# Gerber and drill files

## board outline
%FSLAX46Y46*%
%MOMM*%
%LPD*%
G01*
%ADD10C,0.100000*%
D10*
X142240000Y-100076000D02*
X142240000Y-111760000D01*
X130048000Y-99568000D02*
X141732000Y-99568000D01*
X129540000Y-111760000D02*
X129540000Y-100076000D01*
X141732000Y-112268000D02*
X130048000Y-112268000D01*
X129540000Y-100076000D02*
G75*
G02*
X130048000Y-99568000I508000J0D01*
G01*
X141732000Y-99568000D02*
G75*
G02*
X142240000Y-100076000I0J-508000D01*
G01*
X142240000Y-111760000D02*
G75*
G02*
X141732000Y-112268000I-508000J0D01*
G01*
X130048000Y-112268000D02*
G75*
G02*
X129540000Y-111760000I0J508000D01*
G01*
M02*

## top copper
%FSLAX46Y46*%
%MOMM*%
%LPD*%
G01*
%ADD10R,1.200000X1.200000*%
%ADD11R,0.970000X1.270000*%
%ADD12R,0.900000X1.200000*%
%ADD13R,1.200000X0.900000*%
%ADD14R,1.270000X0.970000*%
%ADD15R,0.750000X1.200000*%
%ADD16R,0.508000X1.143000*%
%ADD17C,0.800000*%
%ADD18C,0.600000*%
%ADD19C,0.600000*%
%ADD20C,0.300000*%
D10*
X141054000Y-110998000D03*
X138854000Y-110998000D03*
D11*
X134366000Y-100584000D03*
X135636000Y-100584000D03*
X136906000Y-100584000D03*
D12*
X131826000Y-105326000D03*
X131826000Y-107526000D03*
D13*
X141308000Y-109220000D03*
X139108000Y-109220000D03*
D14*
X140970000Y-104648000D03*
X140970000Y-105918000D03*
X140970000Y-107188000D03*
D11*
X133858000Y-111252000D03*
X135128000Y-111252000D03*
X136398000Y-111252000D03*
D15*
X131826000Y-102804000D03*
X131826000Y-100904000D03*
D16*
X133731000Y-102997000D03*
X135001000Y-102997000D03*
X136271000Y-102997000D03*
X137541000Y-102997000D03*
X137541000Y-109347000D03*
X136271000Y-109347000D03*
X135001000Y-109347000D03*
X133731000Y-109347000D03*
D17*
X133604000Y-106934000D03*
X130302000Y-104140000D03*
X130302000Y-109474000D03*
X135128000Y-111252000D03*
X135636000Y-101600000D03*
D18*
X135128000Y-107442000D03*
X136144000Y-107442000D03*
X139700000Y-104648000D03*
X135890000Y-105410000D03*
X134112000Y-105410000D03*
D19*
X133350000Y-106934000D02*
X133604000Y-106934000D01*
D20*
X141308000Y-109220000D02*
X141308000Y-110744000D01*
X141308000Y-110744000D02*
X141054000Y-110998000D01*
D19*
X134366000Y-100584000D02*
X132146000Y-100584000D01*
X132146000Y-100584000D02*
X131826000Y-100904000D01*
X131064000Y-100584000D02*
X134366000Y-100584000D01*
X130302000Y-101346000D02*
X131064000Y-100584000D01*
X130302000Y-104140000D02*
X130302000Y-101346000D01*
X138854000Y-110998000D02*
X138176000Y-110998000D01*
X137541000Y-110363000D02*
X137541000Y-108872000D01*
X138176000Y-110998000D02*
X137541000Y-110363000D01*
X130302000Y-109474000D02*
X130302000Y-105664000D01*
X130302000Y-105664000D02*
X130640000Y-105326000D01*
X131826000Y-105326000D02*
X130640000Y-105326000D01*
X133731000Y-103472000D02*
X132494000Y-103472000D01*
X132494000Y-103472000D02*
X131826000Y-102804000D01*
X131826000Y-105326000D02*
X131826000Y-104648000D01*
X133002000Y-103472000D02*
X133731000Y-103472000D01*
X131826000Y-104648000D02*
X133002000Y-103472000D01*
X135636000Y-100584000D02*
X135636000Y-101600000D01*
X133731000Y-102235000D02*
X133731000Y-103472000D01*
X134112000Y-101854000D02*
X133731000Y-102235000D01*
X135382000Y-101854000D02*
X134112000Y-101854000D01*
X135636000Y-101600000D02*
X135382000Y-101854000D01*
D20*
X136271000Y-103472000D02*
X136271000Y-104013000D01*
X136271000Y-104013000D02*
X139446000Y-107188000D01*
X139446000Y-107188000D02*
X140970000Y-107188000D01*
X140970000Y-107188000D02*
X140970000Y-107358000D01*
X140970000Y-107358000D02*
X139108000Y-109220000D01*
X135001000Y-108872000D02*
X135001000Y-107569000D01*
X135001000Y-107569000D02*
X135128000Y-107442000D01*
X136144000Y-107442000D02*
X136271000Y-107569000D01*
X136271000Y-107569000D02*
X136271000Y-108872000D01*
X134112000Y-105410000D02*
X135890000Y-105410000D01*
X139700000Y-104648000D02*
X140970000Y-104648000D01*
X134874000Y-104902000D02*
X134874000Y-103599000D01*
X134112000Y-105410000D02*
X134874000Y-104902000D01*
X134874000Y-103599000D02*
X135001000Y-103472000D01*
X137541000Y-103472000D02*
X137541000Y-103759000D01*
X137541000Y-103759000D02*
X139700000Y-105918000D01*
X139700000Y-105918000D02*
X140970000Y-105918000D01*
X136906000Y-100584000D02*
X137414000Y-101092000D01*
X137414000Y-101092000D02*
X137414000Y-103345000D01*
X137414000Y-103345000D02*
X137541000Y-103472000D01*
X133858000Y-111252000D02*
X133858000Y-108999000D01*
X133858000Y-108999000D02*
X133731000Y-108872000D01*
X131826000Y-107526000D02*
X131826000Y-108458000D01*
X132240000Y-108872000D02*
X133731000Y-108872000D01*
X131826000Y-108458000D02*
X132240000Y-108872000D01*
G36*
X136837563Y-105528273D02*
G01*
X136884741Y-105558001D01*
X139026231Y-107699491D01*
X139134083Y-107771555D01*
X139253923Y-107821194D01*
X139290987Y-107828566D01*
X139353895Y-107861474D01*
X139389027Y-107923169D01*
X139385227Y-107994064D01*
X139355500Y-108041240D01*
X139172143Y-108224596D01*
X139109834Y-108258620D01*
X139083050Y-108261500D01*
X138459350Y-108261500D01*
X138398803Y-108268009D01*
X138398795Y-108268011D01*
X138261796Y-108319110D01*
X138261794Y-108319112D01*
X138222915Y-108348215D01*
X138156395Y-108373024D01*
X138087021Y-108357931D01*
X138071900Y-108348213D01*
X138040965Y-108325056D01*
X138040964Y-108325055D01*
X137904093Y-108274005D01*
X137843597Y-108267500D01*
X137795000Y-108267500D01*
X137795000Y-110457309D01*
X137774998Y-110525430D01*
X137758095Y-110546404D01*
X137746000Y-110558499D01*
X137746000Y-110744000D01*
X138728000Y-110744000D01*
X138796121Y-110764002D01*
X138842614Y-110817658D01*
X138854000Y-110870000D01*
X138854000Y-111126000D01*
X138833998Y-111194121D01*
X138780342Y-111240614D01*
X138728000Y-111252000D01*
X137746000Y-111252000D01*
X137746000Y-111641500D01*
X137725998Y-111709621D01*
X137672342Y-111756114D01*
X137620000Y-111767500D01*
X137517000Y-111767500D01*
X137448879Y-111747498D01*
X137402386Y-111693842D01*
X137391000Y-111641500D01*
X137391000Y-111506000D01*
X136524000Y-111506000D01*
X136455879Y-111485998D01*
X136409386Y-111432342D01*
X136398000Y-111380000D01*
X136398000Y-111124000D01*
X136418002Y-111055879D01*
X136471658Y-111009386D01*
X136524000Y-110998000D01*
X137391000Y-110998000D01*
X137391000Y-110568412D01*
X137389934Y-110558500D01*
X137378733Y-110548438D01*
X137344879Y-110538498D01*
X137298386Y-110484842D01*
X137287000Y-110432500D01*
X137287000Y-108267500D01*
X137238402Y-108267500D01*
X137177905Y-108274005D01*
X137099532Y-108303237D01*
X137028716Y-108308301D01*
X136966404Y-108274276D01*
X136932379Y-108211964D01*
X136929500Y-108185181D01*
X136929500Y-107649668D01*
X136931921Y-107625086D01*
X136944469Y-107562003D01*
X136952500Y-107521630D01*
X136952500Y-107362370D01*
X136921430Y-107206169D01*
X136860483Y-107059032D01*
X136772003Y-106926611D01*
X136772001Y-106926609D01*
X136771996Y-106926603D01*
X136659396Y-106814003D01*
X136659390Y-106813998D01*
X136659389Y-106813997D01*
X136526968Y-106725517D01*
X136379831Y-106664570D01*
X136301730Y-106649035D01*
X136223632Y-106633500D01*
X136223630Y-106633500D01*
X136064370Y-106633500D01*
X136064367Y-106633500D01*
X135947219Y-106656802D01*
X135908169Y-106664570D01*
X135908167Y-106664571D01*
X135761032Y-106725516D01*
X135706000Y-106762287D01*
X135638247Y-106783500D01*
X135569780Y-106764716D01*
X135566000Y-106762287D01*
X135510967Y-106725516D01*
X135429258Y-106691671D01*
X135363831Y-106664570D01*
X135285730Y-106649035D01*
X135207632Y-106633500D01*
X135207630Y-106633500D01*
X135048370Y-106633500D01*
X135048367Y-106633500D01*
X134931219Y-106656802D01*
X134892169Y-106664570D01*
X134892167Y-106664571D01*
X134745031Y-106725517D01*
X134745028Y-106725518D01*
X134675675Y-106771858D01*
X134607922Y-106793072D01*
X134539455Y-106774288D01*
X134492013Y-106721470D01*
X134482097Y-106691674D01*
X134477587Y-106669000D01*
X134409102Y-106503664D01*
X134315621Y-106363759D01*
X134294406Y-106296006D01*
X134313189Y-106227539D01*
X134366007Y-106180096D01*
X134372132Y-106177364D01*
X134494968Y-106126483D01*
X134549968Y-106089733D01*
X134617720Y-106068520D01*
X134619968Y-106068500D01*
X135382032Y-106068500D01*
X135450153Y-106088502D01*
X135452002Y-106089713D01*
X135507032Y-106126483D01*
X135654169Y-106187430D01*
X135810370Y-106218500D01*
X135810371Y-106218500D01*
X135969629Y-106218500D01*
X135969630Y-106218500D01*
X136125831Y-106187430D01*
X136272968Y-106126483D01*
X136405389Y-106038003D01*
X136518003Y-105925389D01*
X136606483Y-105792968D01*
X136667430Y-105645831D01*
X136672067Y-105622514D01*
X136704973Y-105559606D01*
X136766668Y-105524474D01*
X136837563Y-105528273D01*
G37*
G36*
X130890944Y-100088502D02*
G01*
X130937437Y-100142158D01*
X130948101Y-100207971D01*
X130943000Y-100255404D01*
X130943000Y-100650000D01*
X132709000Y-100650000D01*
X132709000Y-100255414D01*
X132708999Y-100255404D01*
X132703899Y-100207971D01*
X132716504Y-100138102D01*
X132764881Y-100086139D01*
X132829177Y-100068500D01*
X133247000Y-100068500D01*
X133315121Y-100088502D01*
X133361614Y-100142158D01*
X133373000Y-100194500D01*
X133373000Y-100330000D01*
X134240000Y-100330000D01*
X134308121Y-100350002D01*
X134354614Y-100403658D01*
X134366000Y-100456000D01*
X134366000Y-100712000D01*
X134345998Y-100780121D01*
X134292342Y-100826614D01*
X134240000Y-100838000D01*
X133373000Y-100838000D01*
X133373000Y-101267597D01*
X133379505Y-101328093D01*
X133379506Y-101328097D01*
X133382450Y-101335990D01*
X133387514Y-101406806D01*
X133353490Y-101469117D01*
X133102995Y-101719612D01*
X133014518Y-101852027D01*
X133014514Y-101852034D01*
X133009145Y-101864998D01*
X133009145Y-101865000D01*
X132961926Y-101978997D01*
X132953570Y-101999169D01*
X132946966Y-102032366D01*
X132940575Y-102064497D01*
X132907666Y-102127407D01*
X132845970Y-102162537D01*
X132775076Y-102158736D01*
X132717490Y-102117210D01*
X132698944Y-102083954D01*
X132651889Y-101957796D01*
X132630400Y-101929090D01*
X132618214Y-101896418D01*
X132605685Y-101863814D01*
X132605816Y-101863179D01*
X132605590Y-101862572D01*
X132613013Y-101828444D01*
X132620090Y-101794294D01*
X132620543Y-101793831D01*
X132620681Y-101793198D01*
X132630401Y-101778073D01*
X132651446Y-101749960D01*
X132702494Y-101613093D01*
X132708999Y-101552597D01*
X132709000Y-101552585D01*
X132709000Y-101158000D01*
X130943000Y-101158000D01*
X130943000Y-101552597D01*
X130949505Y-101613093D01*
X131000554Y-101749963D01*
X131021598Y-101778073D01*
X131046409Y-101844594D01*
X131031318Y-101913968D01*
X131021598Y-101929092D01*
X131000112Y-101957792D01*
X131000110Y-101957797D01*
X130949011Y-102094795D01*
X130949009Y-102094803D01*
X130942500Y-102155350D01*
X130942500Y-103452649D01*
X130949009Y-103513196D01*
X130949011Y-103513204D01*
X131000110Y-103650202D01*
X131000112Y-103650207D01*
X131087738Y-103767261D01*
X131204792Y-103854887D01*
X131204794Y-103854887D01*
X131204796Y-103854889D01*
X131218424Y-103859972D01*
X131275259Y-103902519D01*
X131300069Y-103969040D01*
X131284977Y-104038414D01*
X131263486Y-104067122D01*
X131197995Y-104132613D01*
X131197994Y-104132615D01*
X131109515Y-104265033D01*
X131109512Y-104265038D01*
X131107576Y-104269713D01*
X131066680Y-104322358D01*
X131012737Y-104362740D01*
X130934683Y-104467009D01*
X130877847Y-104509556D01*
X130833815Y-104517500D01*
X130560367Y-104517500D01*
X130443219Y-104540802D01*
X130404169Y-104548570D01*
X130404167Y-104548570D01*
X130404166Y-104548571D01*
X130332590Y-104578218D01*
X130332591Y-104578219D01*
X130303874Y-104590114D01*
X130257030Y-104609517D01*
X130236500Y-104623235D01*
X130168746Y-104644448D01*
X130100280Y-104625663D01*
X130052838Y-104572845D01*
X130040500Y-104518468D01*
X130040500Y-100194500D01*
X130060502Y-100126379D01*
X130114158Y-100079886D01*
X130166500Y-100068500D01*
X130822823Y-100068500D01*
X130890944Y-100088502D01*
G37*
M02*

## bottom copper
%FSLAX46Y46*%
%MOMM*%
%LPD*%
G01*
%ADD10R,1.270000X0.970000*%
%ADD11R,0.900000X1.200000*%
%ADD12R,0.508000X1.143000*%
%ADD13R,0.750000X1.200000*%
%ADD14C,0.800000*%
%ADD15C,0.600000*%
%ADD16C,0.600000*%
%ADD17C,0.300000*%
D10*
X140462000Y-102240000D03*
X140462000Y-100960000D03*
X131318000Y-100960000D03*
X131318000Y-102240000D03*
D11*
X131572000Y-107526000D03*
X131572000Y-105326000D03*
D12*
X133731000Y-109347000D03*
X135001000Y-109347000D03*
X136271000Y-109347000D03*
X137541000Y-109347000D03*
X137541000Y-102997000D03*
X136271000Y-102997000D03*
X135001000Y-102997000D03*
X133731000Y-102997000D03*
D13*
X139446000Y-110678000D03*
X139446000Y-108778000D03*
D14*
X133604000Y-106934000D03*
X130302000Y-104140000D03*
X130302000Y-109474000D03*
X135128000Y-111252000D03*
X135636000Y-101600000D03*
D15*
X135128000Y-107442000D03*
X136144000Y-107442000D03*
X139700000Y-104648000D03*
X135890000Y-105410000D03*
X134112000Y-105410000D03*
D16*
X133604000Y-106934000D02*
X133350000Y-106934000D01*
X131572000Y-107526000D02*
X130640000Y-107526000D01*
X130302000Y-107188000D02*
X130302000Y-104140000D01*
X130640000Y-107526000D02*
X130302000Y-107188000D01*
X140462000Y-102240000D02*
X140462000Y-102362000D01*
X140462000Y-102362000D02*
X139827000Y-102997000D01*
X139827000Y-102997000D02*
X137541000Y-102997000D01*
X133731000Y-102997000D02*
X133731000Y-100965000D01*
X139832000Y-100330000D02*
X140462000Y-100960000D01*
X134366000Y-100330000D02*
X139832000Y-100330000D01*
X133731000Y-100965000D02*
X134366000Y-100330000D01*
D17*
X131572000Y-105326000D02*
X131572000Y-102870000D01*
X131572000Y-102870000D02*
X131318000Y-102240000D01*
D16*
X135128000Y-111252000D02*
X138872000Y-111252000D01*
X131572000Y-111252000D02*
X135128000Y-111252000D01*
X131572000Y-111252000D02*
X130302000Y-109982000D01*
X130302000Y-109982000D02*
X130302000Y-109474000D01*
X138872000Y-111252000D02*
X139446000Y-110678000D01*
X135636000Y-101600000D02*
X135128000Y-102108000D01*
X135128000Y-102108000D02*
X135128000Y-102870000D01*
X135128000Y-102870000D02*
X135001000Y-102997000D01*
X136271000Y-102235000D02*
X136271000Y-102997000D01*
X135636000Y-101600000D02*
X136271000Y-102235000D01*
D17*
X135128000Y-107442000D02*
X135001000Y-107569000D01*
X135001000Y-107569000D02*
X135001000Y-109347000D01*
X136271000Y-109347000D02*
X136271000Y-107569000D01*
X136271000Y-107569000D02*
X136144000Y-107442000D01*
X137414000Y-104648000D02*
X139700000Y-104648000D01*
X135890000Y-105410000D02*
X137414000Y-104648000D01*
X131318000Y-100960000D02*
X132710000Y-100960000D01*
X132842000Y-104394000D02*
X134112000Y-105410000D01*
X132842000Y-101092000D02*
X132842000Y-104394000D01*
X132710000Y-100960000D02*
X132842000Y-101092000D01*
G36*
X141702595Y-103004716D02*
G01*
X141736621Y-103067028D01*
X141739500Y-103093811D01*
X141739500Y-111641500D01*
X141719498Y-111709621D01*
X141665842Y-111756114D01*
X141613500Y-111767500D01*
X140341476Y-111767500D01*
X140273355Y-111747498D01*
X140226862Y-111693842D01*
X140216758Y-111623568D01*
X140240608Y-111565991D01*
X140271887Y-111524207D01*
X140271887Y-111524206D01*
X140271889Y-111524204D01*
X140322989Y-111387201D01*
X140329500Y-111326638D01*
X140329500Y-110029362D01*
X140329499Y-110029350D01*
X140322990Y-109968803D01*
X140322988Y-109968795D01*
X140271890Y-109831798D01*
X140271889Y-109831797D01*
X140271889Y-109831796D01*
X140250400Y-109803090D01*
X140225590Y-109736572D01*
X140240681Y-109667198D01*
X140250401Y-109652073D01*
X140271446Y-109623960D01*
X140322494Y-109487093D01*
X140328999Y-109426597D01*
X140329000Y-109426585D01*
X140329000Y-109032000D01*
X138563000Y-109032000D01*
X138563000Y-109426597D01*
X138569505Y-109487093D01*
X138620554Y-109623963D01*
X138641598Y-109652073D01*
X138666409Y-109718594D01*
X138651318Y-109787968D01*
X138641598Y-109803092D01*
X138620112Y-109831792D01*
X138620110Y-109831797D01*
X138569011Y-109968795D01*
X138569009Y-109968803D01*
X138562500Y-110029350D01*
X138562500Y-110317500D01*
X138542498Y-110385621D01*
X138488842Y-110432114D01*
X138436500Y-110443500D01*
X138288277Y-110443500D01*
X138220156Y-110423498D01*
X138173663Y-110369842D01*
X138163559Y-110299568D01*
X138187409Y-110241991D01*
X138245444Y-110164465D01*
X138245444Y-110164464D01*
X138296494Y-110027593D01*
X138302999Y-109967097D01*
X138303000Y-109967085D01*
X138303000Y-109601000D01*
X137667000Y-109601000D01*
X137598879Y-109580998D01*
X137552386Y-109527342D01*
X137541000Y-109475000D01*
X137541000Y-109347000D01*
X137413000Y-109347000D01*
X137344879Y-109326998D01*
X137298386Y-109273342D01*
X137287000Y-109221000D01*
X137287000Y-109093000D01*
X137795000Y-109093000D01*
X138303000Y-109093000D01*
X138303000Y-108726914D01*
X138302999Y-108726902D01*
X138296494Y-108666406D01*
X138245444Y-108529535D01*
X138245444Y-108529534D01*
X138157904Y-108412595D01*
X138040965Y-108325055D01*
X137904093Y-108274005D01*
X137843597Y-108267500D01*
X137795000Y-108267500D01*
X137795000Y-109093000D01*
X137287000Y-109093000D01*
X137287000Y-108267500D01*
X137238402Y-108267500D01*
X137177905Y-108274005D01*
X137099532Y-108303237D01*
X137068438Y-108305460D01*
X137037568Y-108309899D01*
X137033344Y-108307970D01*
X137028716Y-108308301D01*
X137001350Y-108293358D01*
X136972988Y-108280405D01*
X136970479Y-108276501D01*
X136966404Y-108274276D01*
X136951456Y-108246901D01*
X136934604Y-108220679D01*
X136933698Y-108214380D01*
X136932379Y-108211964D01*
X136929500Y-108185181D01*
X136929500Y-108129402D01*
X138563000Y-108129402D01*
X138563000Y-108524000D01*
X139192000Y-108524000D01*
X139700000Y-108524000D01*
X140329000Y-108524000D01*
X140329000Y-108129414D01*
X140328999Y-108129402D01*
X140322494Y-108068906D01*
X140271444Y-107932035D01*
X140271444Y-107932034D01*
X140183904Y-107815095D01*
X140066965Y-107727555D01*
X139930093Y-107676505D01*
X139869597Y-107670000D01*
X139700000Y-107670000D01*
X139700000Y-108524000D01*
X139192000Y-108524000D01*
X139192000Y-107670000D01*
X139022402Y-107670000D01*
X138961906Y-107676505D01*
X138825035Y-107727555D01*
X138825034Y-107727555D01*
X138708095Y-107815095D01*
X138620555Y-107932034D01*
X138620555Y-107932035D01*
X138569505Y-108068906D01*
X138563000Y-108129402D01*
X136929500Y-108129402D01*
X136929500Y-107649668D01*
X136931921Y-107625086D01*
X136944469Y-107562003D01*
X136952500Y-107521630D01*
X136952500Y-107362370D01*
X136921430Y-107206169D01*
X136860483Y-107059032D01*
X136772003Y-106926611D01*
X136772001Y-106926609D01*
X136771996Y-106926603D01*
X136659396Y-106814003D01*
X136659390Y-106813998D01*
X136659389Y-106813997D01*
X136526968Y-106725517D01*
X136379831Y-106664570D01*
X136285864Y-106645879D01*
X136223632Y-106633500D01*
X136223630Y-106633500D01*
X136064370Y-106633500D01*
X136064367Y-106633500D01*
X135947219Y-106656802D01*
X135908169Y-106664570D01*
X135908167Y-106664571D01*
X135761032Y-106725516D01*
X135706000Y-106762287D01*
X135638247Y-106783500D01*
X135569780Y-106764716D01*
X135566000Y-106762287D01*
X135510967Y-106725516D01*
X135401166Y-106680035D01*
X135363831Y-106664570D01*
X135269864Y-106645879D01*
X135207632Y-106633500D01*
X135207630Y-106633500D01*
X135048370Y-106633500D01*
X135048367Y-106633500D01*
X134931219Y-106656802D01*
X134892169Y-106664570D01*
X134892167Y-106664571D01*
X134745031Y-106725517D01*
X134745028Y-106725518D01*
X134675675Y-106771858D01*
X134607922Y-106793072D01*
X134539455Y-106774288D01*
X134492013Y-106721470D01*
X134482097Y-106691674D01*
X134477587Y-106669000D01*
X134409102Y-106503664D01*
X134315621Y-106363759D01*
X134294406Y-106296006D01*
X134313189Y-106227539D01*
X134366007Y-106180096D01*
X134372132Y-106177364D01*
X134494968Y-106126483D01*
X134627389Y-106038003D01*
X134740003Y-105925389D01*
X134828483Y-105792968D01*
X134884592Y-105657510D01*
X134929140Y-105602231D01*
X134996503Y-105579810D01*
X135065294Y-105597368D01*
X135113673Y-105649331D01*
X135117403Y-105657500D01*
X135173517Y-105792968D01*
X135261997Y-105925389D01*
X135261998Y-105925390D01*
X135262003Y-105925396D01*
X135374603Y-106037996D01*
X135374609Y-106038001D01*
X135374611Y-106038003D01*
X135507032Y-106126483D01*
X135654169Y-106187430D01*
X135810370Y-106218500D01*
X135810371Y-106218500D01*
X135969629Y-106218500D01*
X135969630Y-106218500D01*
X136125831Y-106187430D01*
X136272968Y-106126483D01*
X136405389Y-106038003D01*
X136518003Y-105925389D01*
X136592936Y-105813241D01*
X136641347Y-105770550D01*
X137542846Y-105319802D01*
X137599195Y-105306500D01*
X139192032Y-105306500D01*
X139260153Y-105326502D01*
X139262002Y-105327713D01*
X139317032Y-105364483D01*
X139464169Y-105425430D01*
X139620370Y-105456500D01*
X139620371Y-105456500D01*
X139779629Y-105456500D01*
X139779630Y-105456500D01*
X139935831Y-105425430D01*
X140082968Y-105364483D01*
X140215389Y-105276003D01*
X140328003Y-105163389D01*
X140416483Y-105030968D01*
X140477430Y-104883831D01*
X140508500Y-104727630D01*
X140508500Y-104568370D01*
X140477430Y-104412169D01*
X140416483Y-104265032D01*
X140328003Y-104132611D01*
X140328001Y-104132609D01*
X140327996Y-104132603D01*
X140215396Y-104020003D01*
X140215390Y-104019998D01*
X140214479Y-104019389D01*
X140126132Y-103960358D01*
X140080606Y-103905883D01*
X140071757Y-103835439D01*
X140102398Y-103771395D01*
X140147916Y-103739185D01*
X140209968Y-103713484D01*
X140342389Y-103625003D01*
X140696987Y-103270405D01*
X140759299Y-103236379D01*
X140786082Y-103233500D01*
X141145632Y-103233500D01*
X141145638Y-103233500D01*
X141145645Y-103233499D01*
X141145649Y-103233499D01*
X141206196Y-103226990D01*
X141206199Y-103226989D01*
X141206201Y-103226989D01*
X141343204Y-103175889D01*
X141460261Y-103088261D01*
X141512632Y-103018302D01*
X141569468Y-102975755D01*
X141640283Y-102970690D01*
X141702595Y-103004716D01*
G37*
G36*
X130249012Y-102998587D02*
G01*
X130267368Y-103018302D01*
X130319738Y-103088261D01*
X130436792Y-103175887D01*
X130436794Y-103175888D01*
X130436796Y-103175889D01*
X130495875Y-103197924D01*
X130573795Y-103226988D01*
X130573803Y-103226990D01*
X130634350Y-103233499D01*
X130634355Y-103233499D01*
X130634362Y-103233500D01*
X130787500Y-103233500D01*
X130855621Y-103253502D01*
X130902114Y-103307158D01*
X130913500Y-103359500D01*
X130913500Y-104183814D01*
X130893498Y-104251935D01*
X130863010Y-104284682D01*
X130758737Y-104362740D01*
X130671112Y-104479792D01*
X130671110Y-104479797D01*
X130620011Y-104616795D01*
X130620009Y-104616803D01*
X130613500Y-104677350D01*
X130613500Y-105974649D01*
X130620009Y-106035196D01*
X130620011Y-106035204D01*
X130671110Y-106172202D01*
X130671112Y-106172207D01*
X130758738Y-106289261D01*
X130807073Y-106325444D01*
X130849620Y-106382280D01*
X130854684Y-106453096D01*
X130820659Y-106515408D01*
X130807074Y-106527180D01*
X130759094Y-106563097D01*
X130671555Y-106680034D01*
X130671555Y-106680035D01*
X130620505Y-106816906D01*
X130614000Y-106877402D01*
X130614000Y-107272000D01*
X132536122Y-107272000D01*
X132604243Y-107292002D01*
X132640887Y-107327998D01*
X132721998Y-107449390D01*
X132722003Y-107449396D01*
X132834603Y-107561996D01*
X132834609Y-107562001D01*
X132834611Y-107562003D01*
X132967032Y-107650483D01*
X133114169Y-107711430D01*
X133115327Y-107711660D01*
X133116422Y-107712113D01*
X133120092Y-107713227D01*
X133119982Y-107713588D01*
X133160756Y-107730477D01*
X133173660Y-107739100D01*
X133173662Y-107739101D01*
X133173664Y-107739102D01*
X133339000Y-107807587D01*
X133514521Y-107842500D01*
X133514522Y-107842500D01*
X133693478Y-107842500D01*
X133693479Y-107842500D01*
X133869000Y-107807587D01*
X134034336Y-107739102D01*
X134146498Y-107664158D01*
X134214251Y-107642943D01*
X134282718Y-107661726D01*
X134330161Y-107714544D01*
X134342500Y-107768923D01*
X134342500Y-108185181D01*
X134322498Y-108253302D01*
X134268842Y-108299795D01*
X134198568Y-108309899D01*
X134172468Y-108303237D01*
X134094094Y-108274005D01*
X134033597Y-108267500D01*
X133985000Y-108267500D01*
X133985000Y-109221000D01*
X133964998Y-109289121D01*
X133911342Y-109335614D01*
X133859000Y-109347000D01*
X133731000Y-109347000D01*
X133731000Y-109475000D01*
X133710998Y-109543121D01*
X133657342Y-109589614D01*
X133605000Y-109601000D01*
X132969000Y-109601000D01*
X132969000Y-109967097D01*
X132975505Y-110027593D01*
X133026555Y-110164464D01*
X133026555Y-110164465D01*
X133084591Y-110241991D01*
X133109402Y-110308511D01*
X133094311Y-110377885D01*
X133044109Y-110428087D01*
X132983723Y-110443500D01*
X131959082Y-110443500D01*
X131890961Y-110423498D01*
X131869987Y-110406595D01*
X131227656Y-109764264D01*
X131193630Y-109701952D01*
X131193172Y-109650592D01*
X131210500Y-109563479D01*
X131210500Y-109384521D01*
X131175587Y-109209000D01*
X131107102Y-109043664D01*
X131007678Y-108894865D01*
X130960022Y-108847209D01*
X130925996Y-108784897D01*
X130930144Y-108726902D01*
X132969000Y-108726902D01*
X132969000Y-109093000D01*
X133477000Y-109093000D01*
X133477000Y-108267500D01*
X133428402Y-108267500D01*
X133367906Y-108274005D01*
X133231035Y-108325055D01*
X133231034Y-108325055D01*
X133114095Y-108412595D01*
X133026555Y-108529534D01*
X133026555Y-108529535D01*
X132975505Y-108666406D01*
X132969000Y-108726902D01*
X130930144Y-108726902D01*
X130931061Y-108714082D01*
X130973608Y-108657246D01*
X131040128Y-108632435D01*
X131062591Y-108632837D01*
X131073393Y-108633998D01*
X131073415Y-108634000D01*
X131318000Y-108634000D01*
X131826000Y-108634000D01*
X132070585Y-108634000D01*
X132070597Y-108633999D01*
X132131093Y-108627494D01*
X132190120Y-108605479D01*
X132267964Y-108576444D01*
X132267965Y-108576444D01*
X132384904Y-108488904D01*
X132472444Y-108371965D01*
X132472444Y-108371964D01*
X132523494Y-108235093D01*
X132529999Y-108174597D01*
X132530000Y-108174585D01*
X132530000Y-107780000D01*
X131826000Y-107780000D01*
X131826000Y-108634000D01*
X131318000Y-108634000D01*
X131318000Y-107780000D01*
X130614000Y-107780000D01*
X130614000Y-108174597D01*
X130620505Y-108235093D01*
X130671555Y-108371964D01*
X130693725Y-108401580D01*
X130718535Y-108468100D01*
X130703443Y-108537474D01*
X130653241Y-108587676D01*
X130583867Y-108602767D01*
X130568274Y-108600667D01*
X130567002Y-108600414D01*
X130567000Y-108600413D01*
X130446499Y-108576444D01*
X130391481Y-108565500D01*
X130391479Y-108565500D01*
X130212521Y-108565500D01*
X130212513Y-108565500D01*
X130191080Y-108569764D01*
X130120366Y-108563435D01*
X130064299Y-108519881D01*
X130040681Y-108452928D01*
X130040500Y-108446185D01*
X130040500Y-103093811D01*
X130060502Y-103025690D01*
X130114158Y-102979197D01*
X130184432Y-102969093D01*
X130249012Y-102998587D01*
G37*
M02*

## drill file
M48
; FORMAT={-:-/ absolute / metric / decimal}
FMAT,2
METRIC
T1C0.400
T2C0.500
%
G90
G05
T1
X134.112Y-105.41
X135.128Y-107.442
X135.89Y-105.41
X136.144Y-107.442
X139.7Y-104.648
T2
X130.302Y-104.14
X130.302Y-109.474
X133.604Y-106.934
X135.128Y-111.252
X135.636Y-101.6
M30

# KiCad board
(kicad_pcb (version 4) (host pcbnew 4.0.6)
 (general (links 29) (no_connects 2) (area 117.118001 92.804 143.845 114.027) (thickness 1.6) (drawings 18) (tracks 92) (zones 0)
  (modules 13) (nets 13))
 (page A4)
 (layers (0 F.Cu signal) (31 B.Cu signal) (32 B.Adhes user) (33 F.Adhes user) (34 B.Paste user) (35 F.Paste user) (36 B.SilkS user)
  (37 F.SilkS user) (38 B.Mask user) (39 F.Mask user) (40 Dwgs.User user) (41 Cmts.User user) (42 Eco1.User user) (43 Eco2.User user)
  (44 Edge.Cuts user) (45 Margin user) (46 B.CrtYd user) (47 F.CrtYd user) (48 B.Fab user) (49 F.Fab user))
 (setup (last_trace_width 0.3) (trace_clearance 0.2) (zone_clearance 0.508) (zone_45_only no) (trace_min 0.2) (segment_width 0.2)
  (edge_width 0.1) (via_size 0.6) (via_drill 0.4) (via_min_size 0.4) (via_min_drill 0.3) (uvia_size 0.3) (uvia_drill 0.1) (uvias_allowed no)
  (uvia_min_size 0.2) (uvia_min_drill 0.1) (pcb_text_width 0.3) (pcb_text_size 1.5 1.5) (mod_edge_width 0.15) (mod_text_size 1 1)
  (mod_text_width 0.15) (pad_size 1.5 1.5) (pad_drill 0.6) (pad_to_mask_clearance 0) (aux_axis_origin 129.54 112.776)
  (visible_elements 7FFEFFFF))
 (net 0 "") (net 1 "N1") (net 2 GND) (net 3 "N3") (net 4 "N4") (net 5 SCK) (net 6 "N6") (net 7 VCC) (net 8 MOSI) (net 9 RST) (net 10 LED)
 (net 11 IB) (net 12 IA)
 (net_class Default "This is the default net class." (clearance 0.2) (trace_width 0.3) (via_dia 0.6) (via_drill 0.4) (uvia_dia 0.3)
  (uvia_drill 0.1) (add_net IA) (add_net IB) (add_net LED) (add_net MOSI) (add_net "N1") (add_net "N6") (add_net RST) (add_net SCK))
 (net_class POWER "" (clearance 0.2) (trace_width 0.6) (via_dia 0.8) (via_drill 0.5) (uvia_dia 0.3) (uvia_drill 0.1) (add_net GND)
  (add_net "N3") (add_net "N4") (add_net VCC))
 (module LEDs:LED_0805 (layer F.Cu) (at 139.954 110.998)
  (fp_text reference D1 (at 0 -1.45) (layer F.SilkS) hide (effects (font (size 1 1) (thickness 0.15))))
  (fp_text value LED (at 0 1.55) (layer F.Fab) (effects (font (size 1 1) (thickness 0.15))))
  (pad 2 smd rect (at 1.1 0 180) (size 1.2 1.2) (layers F.Cu F.Paste F.Mask) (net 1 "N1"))
  (pad 1 smd rect (at -1.1 0 180) (size 1.2 1.2) (layers F.Cu F.Paste F.Mask) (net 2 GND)))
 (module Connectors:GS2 (layer B.Cu) (at 140.462 101.6)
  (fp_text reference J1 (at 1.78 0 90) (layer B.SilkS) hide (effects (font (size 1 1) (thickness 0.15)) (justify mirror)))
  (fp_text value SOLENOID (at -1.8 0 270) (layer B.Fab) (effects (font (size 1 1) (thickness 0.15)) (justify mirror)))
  (pad 1 smd rect (at 0 0.64) (size 1.27 0.97) (layers B.Cu B.Paste B.Mask) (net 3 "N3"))
  (pad 2 smd rect (at 0 -0.64) (size 1.27 0.97) (layers B.Cu B.Paste B.Mask) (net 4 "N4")))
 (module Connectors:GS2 (layer B.Cu) (at 131.318 101.6 180)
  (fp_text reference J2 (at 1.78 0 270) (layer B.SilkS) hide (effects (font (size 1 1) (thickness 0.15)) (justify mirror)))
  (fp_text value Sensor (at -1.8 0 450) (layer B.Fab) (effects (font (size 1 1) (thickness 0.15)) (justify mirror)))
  (pad 1 smd rect (at 0 0.64 180) (size 1.27 0.97) (layers B.Cu B.Paste B.Mask) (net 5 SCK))
  (pad 2 smd rect (at 0 -0.64 180) (size 1.27 0.97) (layers B.Cu B.Paste B.Mask) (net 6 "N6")))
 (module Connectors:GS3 (layer F.Cu) (at 135.636 100.584 90)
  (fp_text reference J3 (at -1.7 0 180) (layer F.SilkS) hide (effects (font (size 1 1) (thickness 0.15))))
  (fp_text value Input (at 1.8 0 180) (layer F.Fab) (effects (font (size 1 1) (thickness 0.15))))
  (pad 1 smd rect (at 0 -1.27 90) (size 1.27 0.97) (layers F.Cu F.Paste F.Mask) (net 2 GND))
  (pad 2 smd rect (at 0 0 90) (size 1.27 0.97) (layers F.Cu F.Paste F.Mask) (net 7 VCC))
  (pad 3 smd rect (at 0 1.27 90) (size 1.27 0.97) (layers F.Cu F.Paste F.Mask) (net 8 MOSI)))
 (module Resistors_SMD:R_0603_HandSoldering (layer F.Cu) (at 131.826 106.426 270)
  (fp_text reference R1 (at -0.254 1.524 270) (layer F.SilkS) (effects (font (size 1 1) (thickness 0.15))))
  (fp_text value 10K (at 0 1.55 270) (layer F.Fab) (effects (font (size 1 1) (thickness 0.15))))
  (pad 1 smd rect (at -1.1 0 270) (size 1.2 0.9) (layers F.Cu F.Paste F.Mask) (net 7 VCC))
  (pad 2 smd rect (at 1.1 0 270) (size 1.2 0.9) (layers F.Cu F.Paste F.Mask) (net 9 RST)))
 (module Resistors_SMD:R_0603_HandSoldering (layer B.Cu) (at 131.572 106.426 90)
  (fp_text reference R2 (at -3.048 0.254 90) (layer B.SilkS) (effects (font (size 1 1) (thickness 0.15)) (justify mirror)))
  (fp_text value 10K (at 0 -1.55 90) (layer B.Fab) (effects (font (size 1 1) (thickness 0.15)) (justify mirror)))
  (pad 1 smd rect (at -1.1 0 90) (size 1.2 0.9) (layers B.Cu B.Paste B.Mask) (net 2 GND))
  (pad 2 smd rect (at 1.1 0 90) (size 1.2 0.9) (layers B.Cu B.Paste B.Mask) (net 6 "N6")))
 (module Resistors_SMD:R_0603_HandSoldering (layer F.Cu) (at 140.208 109.22 180)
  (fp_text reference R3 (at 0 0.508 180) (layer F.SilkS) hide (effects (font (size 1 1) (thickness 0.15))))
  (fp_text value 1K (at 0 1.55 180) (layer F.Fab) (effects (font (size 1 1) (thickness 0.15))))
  (pad 1 smd rect (at -1.1 0 180) (size 1.2 0.9) (layers F.Cu F.Paste F.Mask) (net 1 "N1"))
  (pad 2 smd rect (at 1.1 0 180) (size 1.2 0.9) (layers F.Cu F.Paste F.Mask) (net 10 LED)))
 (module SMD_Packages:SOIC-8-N (layer B.Cu) (at 135.636 106.172)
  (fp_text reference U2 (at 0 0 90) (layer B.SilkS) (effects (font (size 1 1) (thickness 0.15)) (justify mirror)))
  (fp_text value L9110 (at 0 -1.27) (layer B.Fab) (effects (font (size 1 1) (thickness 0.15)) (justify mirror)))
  (pad 8 smd rect (at -1.905 3.175) (size 0.508 1.143) (layers B.Cu B.Paste B.Mask) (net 2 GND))
  (pad 7 smd rect (at -0.635 3.175) (size 0.508 1.143) (layers B.Cu B.Paste B.Mask) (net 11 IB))
  (pad 6 smd rect (at 0.635 3.175) (size 0.508 1.143) (layers B.Cu B.Paste B.Mask) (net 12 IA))
  (pad 5 smd rect (at 1.905 3.175) (size 0.508 1.143) (layers B.Cu B.Paste B.Mask) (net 2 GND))
  (pad 4 smd rect (at 1.905 -3.175) (size 0.508 1.143) (layers B.Cu B.Paste B.Mask) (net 3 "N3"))
  (pad 3 smd rect (at 0.635 -3.175) (size 0.508 1.143) (layers B.Cu B.Paste B.Mask) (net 7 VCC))
  (pad 2 smd rect (at -0.635 -3.175) (size 0.508 1.143) (layers B.Cu B.Paste B.Mask) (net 7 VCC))
  (pad 1 smd rect (at -1.905 -3.175) (size 0.508 1.143) (layers B.Cu B.Paste B.Mask) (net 4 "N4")))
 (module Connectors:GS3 (layer F.Cu) (at 140.97 105.918)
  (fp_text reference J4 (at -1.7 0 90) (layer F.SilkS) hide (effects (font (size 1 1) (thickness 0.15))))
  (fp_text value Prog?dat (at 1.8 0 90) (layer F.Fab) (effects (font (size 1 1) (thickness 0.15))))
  (pad 1 smd rect (at 0 -1.27) (size 1.27 0.97) (layers F.Cu F.Paste F.Mask) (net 5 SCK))
  (pad 2 smd rect (at 0 0) (size 1.27 0.97) (layers F.Cu F.Paste F.Mask) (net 8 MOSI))
  (pad 3 smd rect (at 0 1.27) (size 1.27 0.97) (layers F.Cu F.Paste F.Mask) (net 10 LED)))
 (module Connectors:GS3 (layer F.Cu) (at 135.128 111.252 90)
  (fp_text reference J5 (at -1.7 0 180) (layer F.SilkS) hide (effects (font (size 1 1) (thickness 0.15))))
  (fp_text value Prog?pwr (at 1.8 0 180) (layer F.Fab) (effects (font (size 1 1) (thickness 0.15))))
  (pad 1 smd rect (at 0 -1.27 90) (size 1.27 0.97) (layers F.Cu F.Paste F.Mask) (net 9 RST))
  (pad 2 smd rect (at 0 0 90) (size 1.27 0.97) (layers F.Cu F.Paste F.Mask) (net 7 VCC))
  (pad 3 smd rect (at 0 1.27 90) (size 1.27 0.97) (layers F.Cu F.Paste F.Mask) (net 2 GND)))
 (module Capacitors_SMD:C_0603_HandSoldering (layer B.Cu) (at 139.446 109.728 90)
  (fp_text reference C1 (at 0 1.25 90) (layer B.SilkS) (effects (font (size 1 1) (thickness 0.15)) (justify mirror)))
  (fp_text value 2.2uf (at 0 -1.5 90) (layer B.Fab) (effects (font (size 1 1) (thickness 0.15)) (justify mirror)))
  (pad 1 smd rect (at -0.95 0 90) (size 1.2 0.75) (layers B.Cu B.Paste B.Mask) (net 7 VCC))
  (pad 2 smd rect (at 0.95 0 90) (size 1.2 0.75) (layers B.Cu B.Paste B.Mask) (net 2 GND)))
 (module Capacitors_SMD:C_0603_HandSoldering (layer F.Cu) (at 131.826 101.854 90)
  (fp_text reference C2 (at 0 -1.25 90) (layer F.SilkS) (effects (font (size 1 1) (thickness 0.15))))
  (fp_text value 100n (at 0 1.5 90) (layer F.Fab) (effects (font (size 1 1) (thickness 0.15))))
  (pad 1 smd rect (at -0.95 0 90) (size 1.2 0.75) (layers F.Cu F.Paste F.Mask) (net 7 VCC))
  (pad 2 smd rect (at 0.95 0 90) (size 1.2 0.75) (layers F.Cu F.Paste F.Mask) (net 2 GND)))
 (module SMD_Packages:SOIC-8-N (layer F.Cu) (at 135.636 106.172)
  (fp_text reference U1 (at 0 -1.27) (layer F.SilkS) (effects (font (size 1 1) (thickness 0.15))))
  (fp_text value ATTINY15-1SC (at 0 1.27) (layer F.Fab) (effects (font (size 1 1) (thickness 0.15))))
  (pad 8 smd rect (at -1.905 -3.175) (size 0.508 1.143) (layers F.Cu F.Paste F.Mask) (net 7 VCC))
  (pad 7 smd rect (at -0.635 -3.175) (size 0.508 1.143) (layers F.Cu F.Paste F.Mask) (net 5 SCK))
  (pad 6 smd rect (at 0.635 -3.175) (size 0.508 1.143) (layers F.Cu F.Paste F.Mask) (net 10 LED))
  (pad 5 smd rect (at 1.905 -3.175) (size 0.508 1.143) (layers F.Cu F.Paste F.Mask) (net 8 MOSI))
  (pad 4 smd rect (at 1.905 3.175) (size 0.508 1.143) (layers F.Cu F.Paste F.Mask) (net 2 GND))
  (pad 3 smd rect (at 0.635 3.175) (size 0.508 1.143) (layers F.Cu F.Paste F.Mask) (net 12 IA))
  (pad 2 smd rect (at -0.635 3.175) (size 0.508 1.143) (layers F.Cu F.Paste F.Mask) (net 11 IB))
  (pad 1 smd rect (at -1.905 3.175) (size 0.508 1.143) (layers F.Cu F.Paste F.Mask) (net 9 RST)))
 (gr_line (start 142.24 100.076) (end 142.24 111.76) (angle 90) (layer Edge.Cuts) (width 0.1))
 (gr_line (start 130.048 99.568) (end 141.732 99.568) (angle 90) (layer Edge.Cuts) (width 0.1))
 (gr_line (start 129.54 111.76) (end 129.54 100.076) (angle 90) (layer Edge.Cuts) (width 0.1))
 (gr_line (start 141.732 112.268) (end 130.048 112.268) (angle 90) (layer Edge.Cuts) (width 0.1))
 (gr_arc (start 130.048 100.076) (end 129.54 100.076) (angle 90) (layer Edge.Cuts) (width 0.1))
 (gr_arc (start 141.732 100.076) (end 141.732 99.568) (angle 90) (layer Edge.Cuts) (width 0.1))
 (gr_arc (start 141.732 111.76) (end 142.24 111.76) (angle 90) (layer Edge.Cuts) (width 0.1))
 (gr_arc (start 130.048 111.76) (end 130.048 112.268) (angle 90) (layer Edge.Cuts) (width 0.1))
 (segment (start 133.35 106.934) (end 133.604 106.934) (width 0.6) (layer F.Cu) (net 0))
 (segment (start 133.604 106.934) (end 133.35 106.934) (width 0.6) (layer B.Cu) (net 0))
 (via (at 133.604 106.934) (size 0.8) (drill 0.5) (layers F.Cu B.Cu) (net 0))
 (segment (start 141.308 109.22) (end 141.308 110.744) (width 0.3) (layer F.Cu) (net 1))
 (segment (start 141.308 110.744) (end 141.054 110.998) (width 0.3) (layer F.Cu) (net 1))
 (segment (start 134.366 100.584) (end 132.146 100.584) (width 0.6) (layer F.Cu) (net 2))
 (segment (start 132.146 100.584) (end 131.826 100.904) (width 0.6) (layer F.Cu) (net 2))
 (segment (start 131.572 107.526) (end 130.64 107.526) (width 0.6) (layer B.Cu) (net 2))
 (segment (start 131.064 100.584) (end 134.366 100.584) (width 0.6) (layer F.Cu) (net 2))
 (segment (start 130.302 101.346) (end 131.064 100.584) (width 0.6) (layer F.Cu) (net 2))
 (segment (start 130.302 104.14) (end 130.302 101.346) (width 0.6) (layer F.Cu) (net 2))
 (via (at 130.302 104.14) (size 0.8) (drill 0.5) (layers F.Cu B.Cu) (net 2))
 (segment (start 130.302 107.188) (end 130.302 104.14) (width 0.6) (layer B.Cu) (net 2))
 (segment (start 130.64 107.526) (end 130.302 107.188) (width 0.6) (layer B.Cu) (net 2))
 (segment (start 138.854 110.998) (end 138.176 110.998) (width 0.6) (layer F.Cu) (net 2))
 (segment (start 137.541 110.363) (end 137.541 108.872) (width 0.6) (layer F.Cu) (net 2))
 (segment (start 138.176 110.998) (end 137.541 110.363) (width 0.6) (layer F.Cu) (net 2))
 (segment (start 140.462 102.24) (end 140.462 102.362) (width 0.6) (layer B.Cu) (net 3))
 (segment (start 140.462 102.362) (end 139.827 102.997) (width 0.6) (layer B.Cu) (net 3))
 (segment (start 139.827 102.997) (end 137.541 102.997) (width 0.6) (layer B.Cu) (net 3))
 (segment (start 133.731 102.997) (end 133.731 100.965) (width 0.6) (layer B.Cu) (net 4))
 (segment (start 139.832 100.33) (end 140.462 100.96) (width 0.6) (layer B.Cu) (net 4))
 (segment (start 134.366 100.33) (end 139.832 100.33) (width 0.6) (layer B.Cu) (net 4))
 (segment (start 133.731 100.965) (end 134.366 100.33) (width 0.6) (layer B.Cu) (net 4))
 (segment (start 131.572 105.326) (end 131.572 102.87) (width 0.3) (layer B.Cu) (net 6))
 (segment (start 131.572 102.87) (end 131.318 102.24) (width 0.3) (layer B.Cu) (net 6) (status 20))
 (segment (start 135.128 111.252) (end 138.872 111.252) (width 0.6) (layer B.Cu) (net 7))
 (segment (start 131.572 111.252) (end 135.128 111.252) (width 0.6) (layer B.Cu) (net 7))
 (segment (start 131.572 111.252) (end 130.302 109.982) (width 0.6) (layer B.Cu) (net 7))
 (segment (start 130.302 109.982) (end 130.302 109.474) (width 0.6) (layer B.Cu) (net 7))
 (via (at 130.302 109.474) (size 0.8) (drill 0.5) (layers F.Cu B.Cu) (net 7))
 (segment (start 130.302 109.474) (end 130.302 105.664) (width 0.6) (layer F.Cu) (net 7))
 (segment (start 130.302 105.664) (end 130.64 105.326) (width 0.6) (layer F.Cu) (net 7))
 (segment (start 131.826 105.326) (end 130.64 105.326) (width 0.6) (layer F.Cu) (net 7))
 (via (at 135.128 111.252) (size 0.8) (drill 0.5) (layers F.Cu B.Cu) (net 7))
 (segment (start 138.872 111.252) (end 139.446 110.678) (width 0.6) (layer B.Cu) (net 7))
 (segment (start 133.731 103.472) (end 132.494 103.472) (width 0.6) (layer F.Cu) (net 7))
 (segment (start 132.494 103.472) (end 131.826 102.804) (width 0.6) (layer F.Cu) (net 7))
 (segment (start 131.826 105.326) (end 131.826 104.648) (width 0.6) (layer F.Cu) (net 7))
 (segment (start 133.002 103.472) (end 133.731 103.472) (width 0.6) (layer F.Cu) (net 7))
 (segment (start 131.826 104.648) (end 133.002 103.472) (width 0.6) (layer F.Cu) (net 7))
 (segment (start 135.636 101.6) (end 135.128 102.108) (width 0.6) (layer B.Cu) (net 7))
 (segment (start 135.128 102.108) (end 135.128 102.87) (width 0.6) (layer B.Cu) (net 7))
 (segment (start 135.128 102.87) (end 135.001 102.997) (width 0.6) (layer B.Cu) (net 7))
 (segment (start 135.636 100.584) (end 135.636 101.6) (width 0.6) (layer F.Cu) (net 7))
 (via (at 135.636 101.6) (size 0.8) (drill 0.5) (layers F.Cu B.Cu) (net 7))
 (segment (start 136.271 102.235) (end 136.271 102.997) (width 0.6) (layer B.Cu) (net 7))
 (segment (start 135.636 101.6) (end 136.271 102.235) (width 0.6) (layer B.Cu) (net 7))
 (segment (start 133.731 102.235) (end 133.731 103.472) (width 0.6) (layer F.Cu) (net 7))
 (segment (start 134.112 101.854) (end 133.731 102.235) (width 0.6) (layer F.Cu) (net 7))
 (segment (start 135.382 101.854) (end 134.112 101.854) (width 0.6) (layer F.Cu) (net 7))
 (segment (start 135.636 101.6) (end 135.382 101.854) (width 0.6) (layer F.Cu) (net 7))
 (segment (start 136.271 103.472) (end 136.271 104.013) (width 0.3) (layer F.Cu) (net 10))
 (segment (start 136.271 104.013) (end 139.446 107.188) (width 0.3) (layer F.Cu) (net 10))
 (segment (start 139.446 107.188) (end 140.97 107.188) (width 0.3) (layer F.Cu) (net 10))
 (segment (start 140.97 107.188) (end 140.97 107.358) (width 0.3) (layer F.Cu) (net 10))
 (segment (start 140.97 107.358) (end 139.108 109.22) (width 0.3) (layer F.Cu) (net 10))
 (segment (start 135.001 108.872) (end 135.001 107.569) (width 0.3) (layer F.Cu) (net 11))
 (segment (start 135.001 107.569) (end 135.128 107.442) (width 0.3) (layer F.Cu) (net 11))
 (via (at 135.128 107.442) (size 0.6) (drill 0.4) (layers F.Cu B.Cu) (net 11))
 (segment (start 135.128 107.442) (end 135.001 107.569) (width 0.3) (layer B.Cu) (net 11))
 (segment (start 135.001 107.569) (end 135.001 109.347) (width 0.3) (layer B.Cu) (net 11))
 (segment (start 136.271 109.347) (end 136.271 107.569) (width 0.3) (layer B.Cu) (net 12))
 (segment (start 136.271 107.569) (end 136.144 107.442) (width 0.3) (layer B.Cu) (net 12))
 (via (at 136.144 107.442) (size 0.6) (drill 0.4) (layers F.Cu B.Cu) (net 12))
 (segment (start 136.144 107.442) (end 136.271 107.569) (width 0.3) (layer F.Cu) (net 12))
 (segment (start 136.271 107.569) (end 136.271 108.872) (width 0.3) (layer F.Cu) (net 12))
 (segment (start 134.112 105.41) (end 135.89 105.41) (width 0.3) (layer F.Cu) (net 5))
 (segment (start 139.7 104.648) (end 140.97 104.648) (width 0.3) (layer F.Cu) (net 5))
 (via (at 139.7 104.648) (size 0.6) (drill 0.4) (layers F.Cu B.Cu) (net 5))
 (segment (start 137.414 104.648) (end 139.7 104.648) (width 0.3) (layer B.Cu) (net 5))
 (segment (start 135.89 105.41) (end 137.414 104.648) (width 0.3) (layer B.Cu) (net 5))
 (via (at 135.89 105.41) (size 0.6) (drill 0.4) (layers F.Cu B.Cu) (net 5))
 (segment (start 131.318 100.96) (end 132.71 100.96) (width 0.3) (layer B.Cu) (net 5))
 (segment (start 134.874 104.902) (end 134.874 103.599) (width 0.3) (layer F.Cu) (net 5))
 (segment (start 134.112 105.41) (end 134.874 104.902) (width 0.3) (layer F.Cu) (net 5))
 (via (at 134.112 105.41) (size 0.6) (drill 0.4) (layers F.Cu B.Cu) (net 5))
 (segment (start 132.842 104.394) (end 134.112 105.41) (width 0.3) (layer B.Cu) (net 5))
 (segment (start 132.842 101.092) (end 132.842 104.394) (width 0.3) (layer B.Cu) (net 5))
 (segment (start 132.71 100.96) (end 132.842 101.092) (width 0.3) (layer B.Cu) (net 5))
 (segment (start 134.874 103.599) (end 135.001 103.472) (width 0.3) (layer F.Cu) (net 5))
 (segment (start 137.541 103.472) (end 137.541 103.759) (width 0.3) (layer F.Cu) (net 8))
 (segment (start 137.541 103.759) (end 139.7 105.918) (width 0.3) (layer F.Cu) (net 8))
 (segment (start 139.7 105.918) (end 140.97 105.918) (width 0.3) (layer F.Cu) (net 8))
 (segment (start 136.906 100.584) (end 137.414 101.092) (width 0.3) (layer F.Cu) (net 8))
 (segment (start 137.414 101.092) (end 137.414 103.345) (width 0.3) (layer F.Cu) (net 8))
 (segment (start 137.414 103.345) (end 137.541 103.472) (width 0.3) (layer F.Cu) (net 8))
 (segment (start 133.858 111.252) (end 133.858 108.999) (width 0.3) (layer F.Cu) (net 9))
 (segment (start 133.858 108.999) (end 133.731 108.872) (width 0.3) (layer F.Cu) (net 9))
 (segment (start 131.826 107.526) (end 131.826 108.458) (width 0.3) (layer F.Cu) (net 9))
 (segment (start 132.24 108.872) (end 133.731 108.872) (width 0.3) (layer F.Cu) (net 9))
 (segment (start 131.826 108.458) (end 132.24 108.872) (width 0.3) (layer F.Cu) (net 9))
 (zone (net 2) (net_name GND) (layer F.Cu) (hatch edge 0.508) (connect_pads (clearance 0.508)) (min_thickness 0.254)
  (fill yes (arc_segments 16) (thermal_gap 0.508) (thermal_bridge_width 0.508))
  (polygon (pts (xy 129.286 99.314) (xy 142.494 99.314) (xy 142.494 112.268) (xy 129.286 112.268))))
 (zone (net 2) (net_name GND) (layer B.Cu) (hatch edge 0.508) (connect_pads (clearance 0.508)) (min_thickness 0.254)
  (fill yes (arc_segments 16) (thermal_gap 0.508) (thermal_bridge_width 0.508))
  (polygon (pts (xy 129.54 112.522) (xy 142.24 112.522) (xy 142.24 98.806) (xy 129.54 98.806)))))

